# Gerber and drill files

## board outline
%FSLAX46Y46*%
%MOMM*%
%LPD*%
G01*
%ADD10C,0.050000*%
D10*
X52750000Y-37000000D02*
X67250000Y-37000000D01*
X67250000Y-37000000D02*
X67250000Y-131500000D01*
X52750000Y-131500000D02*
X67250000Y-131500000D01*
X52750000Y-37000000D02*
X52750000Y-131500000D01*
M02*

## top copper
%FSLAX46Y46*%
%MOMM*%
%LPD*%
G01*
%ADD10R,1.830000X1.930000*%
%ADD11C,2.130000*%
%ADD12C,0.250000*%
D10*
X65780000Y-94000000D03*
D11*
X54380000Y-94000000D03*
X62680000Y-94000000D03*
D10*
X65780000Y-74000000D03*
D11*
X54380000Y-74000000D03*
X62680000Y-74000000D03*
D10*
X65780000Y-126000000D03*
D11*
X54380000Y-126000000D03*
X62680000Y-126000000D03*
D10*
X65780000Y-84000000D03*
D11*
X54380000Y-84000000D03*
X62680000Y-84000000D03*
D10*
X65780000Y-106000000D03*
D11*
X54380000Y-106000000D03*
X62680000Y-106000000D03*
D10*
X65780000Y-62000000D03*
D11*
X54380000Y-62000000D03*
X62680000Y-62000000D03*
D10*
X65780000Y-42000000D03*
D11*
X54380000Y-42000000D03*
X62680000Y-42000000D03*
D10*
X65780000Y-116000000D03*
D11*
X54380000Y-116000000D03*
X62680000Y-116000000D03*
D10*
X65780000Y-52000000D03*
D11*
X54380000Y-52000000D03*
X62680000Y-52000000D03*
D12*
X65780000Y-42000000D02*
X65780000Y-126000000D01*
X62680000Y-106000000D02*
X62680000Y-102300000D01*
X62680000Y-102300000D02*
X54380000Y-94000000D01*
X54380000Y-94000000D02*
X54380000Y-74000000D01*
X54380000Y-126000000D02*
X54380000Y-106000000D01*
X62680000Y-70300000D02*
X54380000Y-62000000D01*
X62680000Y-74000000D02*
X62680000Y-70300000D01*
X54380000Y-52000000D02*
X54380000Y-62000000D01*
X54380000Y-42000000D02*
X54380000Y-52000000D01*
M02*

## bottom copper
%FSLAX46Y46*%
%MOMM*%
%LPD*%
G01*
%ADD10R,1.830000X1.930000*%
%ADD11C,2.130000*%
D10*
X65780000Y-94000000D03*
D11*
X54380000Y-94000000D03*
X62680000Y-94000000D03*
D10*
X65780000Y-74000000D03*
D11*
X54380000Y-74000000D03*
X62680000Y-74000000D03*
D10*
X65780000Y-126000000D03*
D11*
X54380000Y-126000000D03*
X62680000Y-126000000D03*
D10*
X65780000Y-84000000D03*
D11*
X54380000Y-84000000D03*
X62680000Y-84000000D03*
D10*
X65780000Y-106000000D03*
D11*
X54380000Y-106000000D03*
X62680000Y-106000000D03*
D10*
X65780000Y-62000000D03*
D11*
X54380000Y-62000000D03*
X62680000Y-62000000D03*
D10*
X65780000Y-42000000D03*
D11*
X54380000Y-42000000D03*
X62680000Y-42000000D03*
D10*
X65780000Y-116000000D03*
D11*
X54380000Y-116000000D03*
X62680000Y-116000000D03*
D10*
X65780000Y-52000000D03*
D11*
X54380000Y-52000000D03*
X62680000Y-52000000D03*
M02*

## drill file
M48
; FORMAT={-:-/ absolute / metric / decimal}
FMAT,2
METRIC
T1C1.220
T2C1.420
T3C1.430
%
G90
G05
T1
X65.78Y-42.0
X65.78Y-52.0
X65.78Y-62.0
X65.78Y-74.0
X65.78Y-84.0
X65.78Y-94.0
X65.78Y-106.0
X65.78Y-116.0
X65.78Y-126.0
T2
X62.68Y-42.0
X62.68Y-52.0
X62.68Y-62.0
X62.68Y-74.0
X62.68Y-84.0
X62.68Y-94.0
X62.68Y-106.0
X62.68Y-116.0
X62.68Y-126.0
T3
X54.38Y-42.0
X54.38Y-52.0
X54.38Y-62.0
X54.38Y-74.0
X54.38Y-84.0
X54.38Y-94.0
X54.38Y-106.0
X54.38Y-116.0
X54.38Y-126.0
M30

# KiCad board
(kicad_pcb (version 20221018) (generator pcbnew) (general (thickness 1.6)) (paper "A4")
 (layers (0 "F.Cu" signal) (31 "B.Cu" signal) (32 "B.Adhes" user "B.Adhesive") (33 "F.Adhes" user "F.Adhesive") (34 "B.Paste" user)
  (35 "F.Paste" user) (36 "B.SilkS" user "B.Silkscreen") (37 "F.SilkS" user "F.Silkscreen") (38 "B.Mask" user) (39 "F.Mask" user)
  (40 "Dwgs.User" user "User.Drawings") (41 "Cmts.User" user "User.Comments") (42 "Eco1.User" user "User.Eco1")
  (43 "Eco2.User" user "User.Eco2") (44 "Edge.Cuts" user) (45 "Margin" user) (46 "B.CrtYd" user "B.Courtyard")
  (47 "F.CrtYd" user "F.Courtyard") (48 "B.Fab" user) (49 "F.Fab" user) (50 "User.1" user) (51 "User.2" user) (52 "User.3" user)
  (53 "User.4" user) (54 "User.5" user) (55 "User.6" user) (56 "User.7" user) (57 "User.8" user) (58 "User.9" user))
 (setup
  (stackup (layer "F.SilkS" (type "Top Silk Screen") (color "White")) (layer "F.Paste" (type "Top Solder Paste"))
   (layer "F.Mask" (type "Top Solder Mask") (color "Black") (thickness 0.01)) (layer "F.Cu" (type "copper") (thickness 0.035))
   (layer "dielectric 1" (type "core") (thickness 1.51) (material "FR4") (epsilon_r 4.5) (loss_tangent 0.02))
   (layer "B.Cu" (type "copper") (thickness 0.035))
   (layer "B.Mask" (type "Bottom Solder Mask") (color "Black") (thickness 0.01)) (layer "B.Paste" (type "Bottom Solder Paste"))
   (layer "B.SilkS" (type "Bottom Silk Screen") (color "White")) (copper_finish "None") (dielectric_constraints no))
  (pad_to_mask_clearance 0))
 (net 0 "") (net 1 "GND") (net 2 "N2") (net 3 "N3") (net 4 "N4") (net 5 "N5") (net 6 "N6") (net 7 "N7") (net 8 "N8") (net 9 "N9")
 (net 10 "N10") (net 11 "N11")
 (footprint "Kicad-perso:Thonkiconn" (layer "F.Cu") (at 65.78 94 -90)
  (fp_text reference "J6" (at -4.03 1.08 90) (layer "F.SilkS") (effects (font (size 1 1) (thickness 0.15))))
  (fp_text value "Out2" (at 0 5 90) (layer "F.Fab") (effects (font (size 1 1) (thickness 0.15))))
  (pad "S" thru_hole rect (at 0 0 90) (size 1.93 1.83) (drill 1.22) (layers "*.Cu" "*.Mask") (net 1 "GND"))
  (pad "T" thru_hole circle (at 0 11.4 90) (size 2.13 2.13) (drill 1.43) (layers "*.Cu" "*.Mask") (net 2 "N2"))
  (pad "TN" thru_hole circle (at 0 3.1 90) (size 2.13 2.13) (drill 1.42) (layers "*.Cu" "*.Mask") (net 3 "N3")))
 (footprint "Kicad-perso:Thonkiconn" (layer "F.Cu") (at 65.78 74 -90)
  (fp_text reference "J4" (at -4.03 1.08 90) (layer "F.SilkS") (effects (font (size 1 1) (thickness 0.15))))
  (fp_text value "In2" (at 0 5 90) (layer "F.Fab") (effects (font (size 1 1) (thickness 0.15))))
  (pad "S" thru_hole rect (at 0 0 90) (size 1.93 1.83) (drill 1.22) (layers "*.Cu" "*.Mask") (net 1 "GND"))
  (pad "T" thru_hole circle (at 0 11.4 90) (size 2.13 2.13) (drill 1.43) (layers "*.Cu" "*.Mask") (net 2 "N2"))
  (pad "TN" thru_hole circle (at 0 3.1 90) (size 2.13 2.13) (drill 1.42) (layers "*.Cu" "*.Mask") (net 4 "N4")))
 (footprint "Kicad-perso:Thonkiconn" (layer "F.Cu") (at 65.78 126 -90)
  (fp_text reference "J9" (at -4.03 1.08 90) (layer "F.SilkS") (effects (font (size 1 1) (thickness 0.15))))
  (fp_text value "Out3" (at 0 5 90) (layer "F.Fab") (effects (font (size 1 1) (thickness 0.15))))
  (pad "S" thru_hole rect (at 0 0 90) (size 1.93 1.83) (drill 1.22) (layers "*.Cu" "*.Mask") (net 1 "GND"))
  (pad "T" thru_hole circle (at 0 11.4 90) (size 2.13 2.13) (drill 1.43) (layers "*.Cu" "*.Mask") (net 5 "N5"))
  (pad "TN" thru_hole circle (at 0 3.1 90) (size 2.13 2.13) (drill 1.42) (layers "*.Cu" "*.Mask") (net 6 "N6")))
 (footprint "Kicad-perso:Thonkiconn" (layer "F.Cu") (at 65.78 84 -90)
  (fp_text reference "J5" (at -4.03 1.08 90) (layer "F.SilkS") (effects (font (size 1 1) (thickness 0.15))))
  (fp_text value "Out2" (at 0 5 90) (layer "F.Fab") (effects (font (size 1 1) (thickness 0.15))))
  (pad "S" thru_hole rect (at 0 0 90) (size 1.93 1.83) (drill 1.22) (layers "*.Cu" "*.Mask") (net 1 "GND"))
  (pad "T" thru_hole circle (at 0 11.4 90) (size 2.13 2.13) (drill 1.43) (layers "*.Cu" "*.Mask") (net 2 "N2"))
  (pad "TN" thru_hole circle (at 0 3.1 90) (size 2.13 2.13) (drill 1.42) (layers "*.Cu" "*.Mask") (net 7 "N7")))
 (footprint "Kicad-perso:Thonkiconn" (layer "F.Cu") (at 65.78 106 -90)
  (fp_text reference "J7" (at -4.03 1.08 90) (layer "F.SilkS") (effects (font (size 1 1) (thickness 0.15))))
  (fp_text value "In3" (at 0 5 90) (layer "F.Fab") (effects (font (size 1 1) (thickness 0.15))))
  (pad "S" thru_hole rect (at 0 0 90) (size 1.93 1.83) (drill 1.22) (layers "*.Cu" "*.Mask") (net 1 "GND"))
  (pad "T" thru_hole circle (at 0 11.4 90) (size 2.13 2.13) (drill 1.43) (layers "*.Cu" "*.Mask") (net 5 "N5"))
  (pad "TN" thru_hole circle (at 0 3.1 90) (size 2.13 2.13) (drill 1.42) (layers "*.Cu" "*.Mask") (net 2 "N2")))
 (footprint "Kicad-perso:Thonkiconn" (layer "F.Cu") (at 65.78 62 -90)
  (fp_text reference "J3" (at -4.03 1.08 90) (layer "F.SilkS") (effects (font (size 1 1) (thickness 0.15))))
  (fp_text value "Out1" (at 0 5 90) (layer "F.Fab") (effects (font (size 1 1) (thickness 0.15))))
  (pad "S" thru_hole rect (at 0 0 90) (size 1.93 1.83) (drill 1.22) (layers "*.Cu" "*.Mask") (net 1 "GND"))
  (pad "T" thru_hole circle (at 0 11.4 90) (size 2.13 2.13) (drill 1.43) (layers "*.Cu" "*.Mask") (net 4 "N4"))
  (pad "TN" thru_hole circle (at 0 3.1 90) (size 2.13 2.13) (drill 1.42) (layers "*.Cu" "*.Mask") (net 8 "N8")))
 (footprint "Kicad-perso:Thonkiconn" (layer "F.Cu") (at 65.78 42 -90)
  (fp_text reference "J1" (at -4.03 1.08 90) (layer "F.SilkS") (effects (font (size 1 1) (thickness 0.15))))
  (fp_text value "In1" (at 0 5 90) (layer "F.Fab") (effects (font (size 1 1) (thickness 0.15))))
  (pad "S" thru_hole rect (at 0 0 90) (size 1.93 1.83) (drill 1.22) (layers "*.Cu" "*.Mask") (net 1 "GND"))
  (pad "T" thru_hole circle (at 0 11.4 90) (size 2.13 2.13) (drill 1.43) (layers "*.Cu" "*.Mask") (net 4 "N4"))
  (pad "TN" thru_hole circle (at 0 3.1 90) (size 2.13 2.13) (drill 1.42) (layers "*.Cu" "*.Mask") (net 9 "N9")))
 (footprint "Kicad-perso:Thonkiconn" (layer "F.Cu") (at 65.78 116 -90)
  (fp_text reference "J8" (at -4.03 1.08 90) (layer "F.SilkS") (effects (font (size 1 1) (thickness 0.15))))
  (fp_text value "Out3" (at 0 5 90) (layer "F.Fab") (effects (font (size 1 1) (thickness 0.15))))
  (pad "S" thru_hole rect (at 0 0 90) (size 1.93 1.83) (drill 1.22) (layers "*.Cu" "*.Mask") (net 1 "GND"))
  (pad "T" thru_hole circle (at 0 11.4 90) (size 2.13 2.13) (drill 1.43) (layers "*.Cu" "*.Mask") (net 5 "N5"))
  (pad "TN" thru_hole circle (at 0 3.1 90) (size 2.13 2.13) (drill 1.42) (layers "*.Cu" "*.Mask") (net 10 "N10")))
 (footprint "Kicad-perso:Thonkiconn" (layer "F.Cu") (at 65.78 52 -90)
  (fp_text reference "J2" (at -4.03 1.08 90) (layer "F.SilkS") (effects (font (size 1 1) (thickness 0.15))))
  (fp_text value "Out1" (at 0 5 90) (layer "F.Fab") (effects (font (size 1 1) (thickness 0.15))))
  (pad "S" thru_hole rect (at 0 0 90) (size 1.93 1.83) (drill 1.22) (layers "*.Cu" "*.Mask") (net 1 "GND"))
  (pad "T" thru_hole circle (at 0 11.4 90) (size 2.13 2.13) (drill 1.43) (layers "*.Cu" "*.Mask") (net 4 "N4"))
  (pad "TN" thru_hole circle (at 0 3.1 90) (size 2.13 2.13) (drill 1.42) (layers "*.Cu" "*.Mask") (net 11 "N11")))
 (gr_line (start 52.75 37) (end 67.25 37) (stroke (width 0.05) (type solid)) (layer "Edge.Cuts"))
 (gr_line (start 67.25 37) (end 67.25 131.5) (stroke (width 0.05) (type solid)) (layer "Edge.Cuts"))
 (gr_line (start 52.75 131.5) (end 67.25 131.5) (stroke (width 0.05) (type solid)) (layer "Edge.Cuts"))
 (gr_line (start 52.75 37) (end 52.75 131.5) (stroke (width 0.05) (type solid)) (layer "Edge.Cuts"))
 (segment (start 65.78 42) (end 65.78 126) (width 0.25) (layer "F.Cu") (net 1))
 (segment (start 62.68 106) (end 62.68 102.3) (width 0.25) (layer "F.Cu") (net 2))
 (segment (start 62.68 102.3) (end 54.38 94) (width 0.25) (layer "F.Cu") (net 2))
 (segment (start 54.38 94) (end 54.38 74) (width 0.25) (layer "F.Cu") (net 2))
 (segment (start 54.38 126) (end 54.38 106) (width 0.25) (layer "F.Cu") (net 5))
 (segment (start 62.68 70.3) (end 54.38 62) (width 0.25) (layer "F.Cu") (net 4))
 (segment (start 62.68 74) (end 62.68 70.3) (width 0.25) (layer "F.Cu") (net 4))
 (segment (start 54.38 52) (end 54.38 62) (width 0.25) (layer "F.Cu") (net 4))
 (segment (start 54.38 42) (end 54.38 52) (width 0.25) (layer "F.Cu") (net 4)))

